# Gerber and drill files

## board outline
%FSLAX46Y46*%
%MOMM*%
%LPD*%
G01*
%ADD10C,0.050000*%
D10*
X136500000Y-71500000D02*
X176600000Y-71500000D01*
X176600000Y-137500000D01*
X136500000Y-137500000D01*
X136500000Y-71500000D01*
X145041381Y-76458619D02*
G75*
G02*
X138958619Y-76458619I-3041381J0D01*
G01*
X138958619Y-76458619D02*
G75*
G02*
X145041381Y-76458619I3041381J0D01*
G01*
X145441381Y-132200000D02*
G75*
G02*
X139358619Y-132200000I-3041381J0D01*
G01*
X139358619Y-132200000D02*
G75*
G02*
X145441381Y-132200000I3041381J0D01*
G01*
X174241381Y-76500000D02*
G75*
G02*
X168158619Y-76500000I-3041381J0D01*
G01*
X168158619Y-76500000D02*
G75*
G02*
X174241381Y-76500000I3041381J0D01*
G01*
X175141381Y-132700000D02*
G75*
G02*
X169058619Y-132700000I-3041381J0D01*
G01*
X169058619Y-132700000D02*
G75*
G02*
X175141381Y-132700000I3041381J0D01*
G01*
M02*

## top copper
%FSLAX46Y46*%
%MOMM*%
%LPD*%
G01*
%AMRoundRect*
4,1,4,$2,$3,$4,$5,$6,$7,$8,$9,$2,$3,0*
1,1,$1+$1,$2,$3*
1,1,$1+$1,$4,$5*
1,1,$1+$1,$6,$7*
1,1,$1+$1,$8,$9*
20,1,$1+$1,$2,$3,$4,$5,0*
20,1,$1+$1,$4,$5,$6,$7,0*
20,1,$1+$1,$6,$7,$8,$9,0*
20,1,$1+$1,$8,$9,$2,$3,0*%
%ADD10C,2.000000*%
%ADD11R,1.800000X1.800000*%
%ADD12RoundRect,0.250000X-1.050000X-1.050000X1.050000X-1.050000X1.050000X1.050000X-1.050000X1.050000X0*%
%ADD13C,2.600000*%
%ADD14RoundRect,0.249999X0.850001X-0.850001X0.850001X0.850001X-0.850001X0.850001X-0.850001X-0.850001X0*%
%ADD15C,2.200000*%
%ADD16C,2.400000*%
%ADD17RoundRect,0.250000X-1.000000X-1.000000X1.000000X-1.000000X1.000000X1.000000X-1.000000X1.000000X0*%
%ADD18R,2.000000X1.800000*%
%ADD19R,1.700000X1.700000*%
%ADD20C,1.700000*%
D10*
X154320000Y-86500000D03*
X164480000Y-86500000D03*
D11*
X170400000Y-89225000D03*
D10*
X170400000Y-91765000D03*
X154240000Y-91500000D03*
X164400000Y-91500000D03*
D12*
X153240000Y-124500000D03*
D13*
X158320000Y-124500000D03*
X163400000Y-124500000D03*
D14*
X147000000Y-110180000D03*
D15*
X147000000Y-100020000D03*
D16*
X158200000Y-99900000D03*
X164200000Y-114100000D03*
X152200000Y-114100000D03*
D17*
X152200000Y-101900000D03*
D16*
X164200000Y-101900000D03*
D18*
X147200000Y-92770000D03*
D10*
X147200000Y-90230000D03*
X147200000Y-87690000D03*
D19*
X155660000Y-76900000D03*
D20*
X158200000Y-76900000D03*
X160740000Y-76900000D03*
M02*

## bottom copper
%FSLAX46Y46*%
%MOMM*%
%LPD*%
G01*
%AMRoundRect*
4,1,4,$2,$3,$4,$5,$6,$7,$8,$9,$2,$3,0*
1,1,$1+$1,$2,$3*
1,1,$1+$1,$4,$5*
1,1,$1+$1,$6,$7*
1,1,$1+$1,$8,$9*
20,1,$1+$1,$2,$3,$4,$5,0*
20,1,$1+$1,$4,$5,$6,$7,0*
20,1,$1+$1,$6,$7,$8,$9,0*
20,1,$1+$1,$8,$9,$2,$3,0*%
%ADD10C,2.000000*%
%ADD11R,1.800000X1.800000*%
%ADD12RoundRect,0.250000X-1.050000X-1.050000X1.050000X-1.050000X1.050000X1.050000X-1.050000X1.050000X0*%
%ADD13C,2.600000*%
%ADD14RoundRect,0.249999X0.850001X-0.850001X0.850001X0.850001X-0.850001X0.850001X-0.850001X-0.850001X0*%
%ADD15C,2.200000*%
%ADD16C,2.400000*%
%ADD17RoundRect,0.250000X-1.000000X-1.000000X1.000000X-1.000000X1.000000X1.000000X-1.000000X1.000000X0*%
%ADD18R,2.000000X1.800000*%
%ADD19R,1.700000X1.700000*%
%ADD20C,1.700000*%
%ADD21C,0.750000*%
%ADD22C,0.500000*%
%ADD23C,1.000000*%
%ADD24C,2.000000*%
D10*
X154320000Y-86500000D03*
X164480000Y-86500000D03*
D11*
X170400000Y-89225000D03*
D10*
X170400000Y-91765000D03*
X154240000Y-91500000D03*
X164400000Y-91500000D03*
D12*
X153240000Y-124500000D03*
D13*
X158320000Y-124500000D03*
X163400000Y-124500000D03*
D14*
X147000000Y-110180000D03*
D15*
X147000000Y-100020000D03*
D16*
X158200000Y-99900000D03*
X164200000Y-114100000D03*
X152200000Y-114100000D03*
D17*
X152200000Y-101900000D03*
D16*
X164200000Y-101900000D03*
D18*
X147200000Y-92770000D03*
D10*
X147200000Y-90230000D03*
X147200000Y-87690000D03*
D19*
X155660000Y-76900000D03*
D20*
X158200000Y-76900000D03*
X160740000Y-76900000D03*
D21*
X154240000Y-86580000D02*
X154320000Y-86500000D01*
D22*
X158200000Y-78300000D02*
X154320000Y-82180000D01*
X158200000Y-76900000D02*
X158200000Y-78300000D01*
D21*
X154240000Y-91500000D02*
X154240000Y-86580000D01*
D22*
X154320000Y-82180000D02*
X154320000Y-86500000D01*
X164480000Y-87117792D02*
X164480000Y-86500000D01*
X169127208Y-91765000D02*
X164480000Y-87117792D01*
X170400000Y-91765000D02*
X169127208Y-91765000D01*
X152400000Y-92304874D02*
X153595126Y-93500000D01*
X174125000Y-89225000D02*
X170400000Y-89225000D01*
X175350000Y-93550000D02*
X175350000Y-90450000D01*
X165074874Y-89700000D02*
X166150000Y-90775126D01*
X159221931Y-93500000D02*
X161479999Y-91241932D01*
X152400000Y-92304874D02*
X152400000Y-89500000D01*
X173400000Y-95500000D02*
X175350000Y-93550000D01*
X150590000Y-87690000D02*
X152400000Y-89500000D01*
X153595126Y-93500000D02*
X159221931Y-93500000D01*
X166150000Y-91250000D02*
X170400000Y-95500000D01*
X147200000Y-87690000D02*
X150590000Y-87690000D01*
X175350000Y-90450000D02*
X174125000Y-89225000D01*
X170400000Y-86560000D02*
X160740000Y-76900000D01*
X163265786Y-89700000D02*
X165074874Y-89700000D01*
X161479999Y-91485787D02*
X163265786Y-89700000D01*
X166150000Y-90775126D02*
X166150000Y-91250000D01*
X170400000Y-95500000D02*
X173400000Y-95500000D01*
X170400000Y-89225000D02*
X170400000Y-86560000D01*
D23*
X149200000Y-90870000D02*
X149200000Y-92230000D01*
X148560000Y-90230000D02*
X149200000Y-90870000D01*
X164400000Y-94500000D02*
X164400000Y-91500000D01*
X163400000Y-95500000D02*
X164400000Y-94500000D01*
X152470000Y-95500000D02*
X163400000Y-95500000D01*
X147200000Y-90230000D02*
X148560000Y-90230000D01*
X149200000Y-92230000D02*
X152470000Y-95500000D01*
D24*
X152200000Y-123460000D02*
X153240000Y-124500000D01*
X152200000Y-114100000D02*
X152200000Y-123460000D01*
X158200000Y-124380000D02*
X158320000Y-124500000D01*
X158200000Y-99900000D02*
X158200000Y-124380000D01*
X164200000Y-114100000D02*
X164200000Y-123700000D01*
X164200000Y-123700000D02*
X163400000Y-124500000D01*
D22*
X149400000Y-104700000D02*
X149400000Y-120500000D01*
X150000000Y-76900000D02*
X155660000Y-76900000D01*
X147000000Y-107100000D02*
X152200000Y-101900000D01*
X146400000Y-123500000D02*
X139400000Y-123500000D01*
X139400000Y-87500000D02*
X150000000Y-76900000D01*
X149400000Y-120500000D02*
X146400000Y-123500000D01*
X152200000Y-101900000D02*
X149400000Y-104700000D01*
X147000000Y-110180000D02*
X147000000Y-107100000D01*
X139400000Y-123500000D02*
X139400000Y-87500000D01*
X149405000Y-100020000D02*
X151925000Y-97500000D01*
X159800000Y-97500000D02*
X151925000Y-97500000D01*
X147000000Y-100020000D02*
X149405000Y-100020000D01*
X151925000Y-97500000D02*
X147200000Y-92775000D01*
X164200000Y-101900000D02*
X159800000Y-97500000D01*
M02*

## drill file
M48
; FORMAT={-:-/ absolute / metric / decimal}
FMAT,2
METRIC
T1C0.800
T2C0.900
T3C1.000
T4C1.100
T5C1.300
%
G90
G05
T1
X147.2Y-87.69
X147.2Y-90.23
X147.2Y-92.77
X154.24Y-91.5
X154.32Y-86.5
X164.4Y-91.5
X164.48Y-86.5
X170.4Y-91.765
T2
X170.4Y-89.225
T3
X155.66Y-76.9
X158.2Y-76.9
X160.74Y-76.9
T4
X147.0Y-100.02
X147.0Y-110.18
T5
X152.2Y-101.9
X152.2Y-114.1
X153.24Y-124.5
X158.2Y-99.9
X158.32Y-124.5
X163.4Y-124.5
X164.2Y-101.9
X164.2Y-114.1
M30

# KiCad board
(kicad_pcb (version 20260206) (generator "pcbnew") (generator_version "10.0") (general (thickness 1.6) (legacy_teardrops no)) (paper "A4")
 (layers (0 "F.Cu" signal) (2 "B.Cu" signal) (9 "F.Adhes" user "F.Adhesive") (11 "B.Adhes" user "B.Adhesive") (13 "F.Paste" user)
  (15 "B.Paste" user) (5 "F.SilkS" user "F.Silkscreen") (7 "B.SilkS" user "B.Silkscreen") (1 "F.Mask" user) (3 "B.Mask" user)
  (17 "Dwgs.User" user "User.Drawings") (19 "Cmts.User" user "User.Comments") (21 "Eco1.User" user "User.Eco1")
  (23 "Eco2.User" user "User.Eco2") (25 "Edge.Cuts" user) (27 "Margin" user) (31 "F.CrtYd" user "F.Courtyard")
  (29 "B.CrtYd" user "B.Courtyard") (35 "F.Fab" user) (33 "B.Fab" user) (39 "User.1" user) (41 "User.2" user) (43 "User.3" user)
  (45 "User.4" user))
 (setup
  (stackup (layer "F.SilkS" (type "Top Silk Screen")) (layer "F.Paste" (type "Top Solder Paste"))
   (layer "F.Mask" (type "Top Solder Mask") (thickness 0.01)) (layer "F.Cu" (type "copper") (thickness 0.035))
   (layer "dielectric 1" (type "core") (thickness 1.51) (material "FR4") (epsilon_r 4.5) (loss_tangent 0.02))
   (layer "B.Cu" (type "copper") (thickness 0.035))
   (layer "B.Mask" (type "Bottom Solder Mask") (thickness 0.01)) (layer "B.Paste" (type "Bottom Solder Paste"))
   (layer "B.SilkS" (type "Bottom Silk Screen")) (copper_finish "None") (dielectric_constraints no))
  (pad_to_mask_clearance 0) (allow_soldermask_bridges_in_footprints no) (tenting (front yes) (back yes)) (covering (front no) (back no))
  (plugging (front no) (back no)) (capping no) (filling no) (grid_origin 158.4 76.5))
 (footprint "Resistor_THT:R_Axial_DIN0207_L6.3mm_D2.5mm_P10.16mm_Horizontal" (layer "F.Cu") (at 154.32 86.5)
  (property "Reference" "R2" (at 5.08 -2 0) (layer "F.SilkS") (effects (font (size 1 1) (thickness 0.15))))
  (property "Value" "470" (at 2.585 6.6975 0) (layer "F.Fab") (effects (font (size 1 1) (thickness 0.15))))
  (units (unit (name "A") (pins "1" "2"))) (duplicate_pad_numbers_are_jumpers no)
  (pad "1" thru_hole circle (at 0 0) (size 2 2) (drill 0.8) (layers "*.Cu" "*.Mask") (remove_unused_layers no) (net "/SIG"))
  (pad "2" thru_hole circle (at 10.16 0) (size 2 2) (drill 0.8) (layers "*.Cu" "*.Mask") (remove_unused_layers no) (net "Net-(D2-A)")))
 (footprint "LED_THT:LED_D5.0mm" (layer "F.Cu") (at 170.4 89.225 -90)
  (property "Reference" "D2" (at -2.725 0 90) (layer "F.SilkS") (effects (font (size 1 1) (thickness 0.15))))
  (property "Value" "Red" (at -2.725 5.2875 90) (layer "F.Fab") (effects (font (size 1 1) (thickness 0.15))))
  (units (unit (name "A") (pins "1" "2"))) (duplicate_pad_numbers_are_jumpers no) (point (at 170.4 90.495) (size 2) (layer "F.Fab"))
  (pad "1" thru_hole rect (at 0 0 270) (size 1.8 1.8) (drill 0.9) (layers "*.Cu" "*.Mask") (remove_unused_layers no) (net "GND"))
  (pad "2" thru_hole circle (at 2.54 0 270) (size 2 2) (drill 0.8) (layers "*.Cu" "*.Mask") (remove_unused_layers no) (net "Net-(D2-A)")))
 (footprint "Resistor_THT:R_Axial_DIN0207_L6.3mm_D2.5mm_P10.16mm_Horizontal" (layer "F.Cu") (at 154.24 91.5)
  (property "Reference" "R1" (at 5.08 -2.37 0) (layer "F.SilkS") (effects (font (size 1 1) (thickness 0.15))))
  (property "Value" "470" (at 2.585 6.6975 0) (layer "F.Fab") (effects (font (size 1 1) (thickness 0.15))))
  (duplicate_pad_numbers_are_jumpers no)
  (pad "1" thru_hole circle (at 0 0) (size 2 2) (drill 0.8) (layers "*.Cu" "*.Mask") (remove_unused_layers no) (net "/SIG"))
  (pad "2" thru_hole circle (at 10.16 0) (size 2 2) (drill 0.8) (layers "*.Cu" "*.Mask") (remove_unused_layers no) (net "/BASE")))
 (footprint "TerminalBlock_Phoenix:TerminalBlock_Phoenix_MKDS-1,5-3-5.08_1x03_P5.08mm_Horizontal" (layer "F.Cu") (at 153.24 124.5)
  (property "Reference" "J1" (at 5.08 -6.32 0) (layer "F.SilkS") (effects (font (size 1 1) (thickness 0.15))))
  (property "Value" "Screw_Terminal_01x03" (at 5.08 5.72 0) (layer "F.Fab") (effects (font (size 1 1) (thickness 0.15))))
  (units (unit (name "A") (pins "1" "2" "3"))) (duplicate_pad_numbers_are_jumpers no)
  (pad "1" thru_hole roundrect (at 0 0) (size 2.6 2.6) (drill 1.3) (layers "*.Cu" "*.Mask") (remove_unused_layers no)
   (roundrect_rratio 0.096154) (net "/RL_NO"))
  (pad "2" thru_hole circle (at 5.08 0) (size 2.6 2.6) (drill 1.3) (layers "*.Cu" "*.Mask") (remove_unused_layers no) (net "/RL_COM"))
  (pad "3" thru_hole circle (at 10.16 0) (size 2.6 2.6) (drill 1.3) (layers "*.Cu" "*.Mask") (remove_unused_layers no) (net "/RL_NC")))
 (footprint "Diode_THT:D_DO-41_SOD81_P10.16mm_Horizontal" (layer "F.Cu") (at 147 110.18 90)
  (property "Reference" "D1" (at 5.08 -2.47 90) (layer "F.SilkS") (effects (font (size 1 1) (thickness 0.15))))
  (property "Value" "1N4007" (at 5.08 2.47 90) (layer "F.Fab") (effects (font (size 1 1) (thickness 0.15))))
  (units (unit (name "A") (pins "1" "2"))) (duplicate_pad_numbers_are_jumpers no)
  (pad "1" thru_hole roundrect (at 0 0 90) (size 2.2 2.2) (drill 1.1) (layers "*.Cu" "*.Mask") (remove_unused_layers no)
   (roundrect_rratio 0.113636) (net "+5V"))
  (pad "2" thru_hole circle (at 10.16 0 90) (size 2.2 2.2) (drill 1.1) (layers "*.Cu" "*.Mask") (remove_unused_layers no) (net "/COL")))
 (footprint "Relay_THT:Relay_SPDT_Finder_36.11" (layer "F.Cu") (at 152.2 101.9)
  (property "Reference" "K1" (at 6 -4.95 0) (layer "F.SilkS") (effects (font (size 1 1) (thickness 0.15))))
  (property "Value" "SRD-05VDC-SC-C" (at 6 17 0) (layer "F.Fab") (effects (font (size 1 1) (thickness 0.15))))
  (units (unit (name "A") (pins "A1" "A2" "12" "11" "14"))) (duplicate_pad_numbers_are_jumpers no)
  (pad "11" thru_hole circle (at 6 -2) (size 2.4 2.4) (drill 1.3) (layers "*.Cu" "*.Mask") (remove_unused_layers no) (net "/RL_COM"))
  (pad "12" thru_hole circle (at 12 12.2) (size 2.4 2.4) (drill 1.3) (layers "*.Cu" "*.Mask") (remove_unused_layers no) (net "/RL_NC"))
  (pad "14" thru_hole circle (at 0 12.2) (size 2.4 2.4) (drill 1.3) (layers "*.Cu" "*.Mask") (remove_unused_layers no) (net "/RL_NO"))
  (pad "A1" thru_hole roundrect (at 0 0) (size 2.5 2.5) (drill 1.3) (layers "*.Cu" "*.Mask") (remove_unused_layers no)
   (roundrect_rratio 0.1) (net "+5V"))
  (pad "A2" thru_hole circle (at 12 0) (size 2.4 2.4) (drill 1.3) (layers "*.Cu" "*.Mask") (remove_unused_layers no) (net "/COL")))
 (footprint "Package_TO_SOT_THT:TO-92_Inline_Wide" (layer "F.Cu") (at 147.2 92.77 90)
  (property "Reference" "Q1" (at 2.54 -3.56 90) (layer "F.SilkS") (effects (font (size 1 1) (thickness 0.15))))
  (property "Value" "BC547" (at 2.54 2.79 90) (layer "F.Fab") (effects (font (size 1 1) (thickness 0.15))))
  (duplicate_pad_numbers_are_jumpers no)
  (pad "1" thru_hole rect (at 0 0 90) (size 1.8 2) (drill 0.8) (layers "*.Cu" "*.Mask") (remove_unused_layers no) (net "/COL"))
  (pad "2" thru_hole circle (at 2.54 0 90) (size 2 2) (drill 0.8) (layers "*.Cu" "*.Mask") (remove_unused_layers no) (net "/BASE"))
  (pad "3" thru_hole circle (at 5.08 0 90) (size 2 2) (drill 0.8) (layers "*.Cu" "*.Mask") (remove_unused_layers no) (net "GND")))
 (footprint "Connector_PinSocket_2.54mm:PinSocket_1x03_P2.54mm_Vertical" (layer "F.Cu") (at 155.66 76.9 90)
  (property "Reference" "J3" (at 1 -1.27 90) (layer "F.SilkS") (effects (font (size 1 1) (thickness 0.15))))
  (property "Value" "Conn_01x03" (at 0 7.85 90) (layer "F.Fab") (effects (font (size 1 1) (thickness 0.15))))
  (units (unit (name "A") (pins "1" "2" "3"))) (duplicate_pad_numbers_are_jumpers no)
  (pad "1" thru_hole rect (at 0 0 90) (size 1.7 1.7) (drill 1) (layers "*.Cu" "*.Mask") (remove_unused_layers no) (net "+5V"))
  (pad "2" thru_hole circle (at 0 2.54 90) (size 1.7 1.7) (drill 1) (layers "*.Cu" "*.Mask") (remove_unused_layers no) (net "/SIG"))
  (pad "3" thru_hole circle (at 0 5.08 90) (size 1.7 1.7) (drill 1) (layers "*.Cu" "*.Mask") (remove_unused_layers no) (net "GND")))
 (gr_rect (start 136.5 71.5) (end 176.6 137.5) (stroke (width 0.05) (type default)) (fill no) (layer "Edge.Cuts"))
 (gr_circle (center 142 76.458619) (end 141.5 73.458619) (stroke (width 0.05) (type default)) (fill no) (layer "Edge.Cuts"))
 (gr_circle (center 142.4 132.2) (end 141.9 129.2) (stroke (width 0.05) (type default)) (fill no) (layer "Edge.Cuts"))
 (gr_circle (center 171.2 76.5) (end 170.7 73.5) (stroke (width 0.05) (type default)) (fill no) (layer "Edge.Cuts"))
 (gr_circle (center 172.1 132.7) (end 171.6 129.7) (stroke (width 0.05) (type default)) (fill no) (layer "Edge.Cuts"))
 (segment (start 154.24 86.58) (end 154.32 86.5) (width 0.75) (layer "B.Cu") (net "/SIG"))
 (segment (start 158.2 78.3) (end 154.32 82.18) (width 0.5) (layer "B.Cu") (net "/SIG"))
 (segment (start 158.2 76.9) (end 158.2 78.3) (width 0.5) (layer "B.Cu") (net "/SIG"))
 (segment (start 154.24 91.5) (end 154.24 86.58) (width 0.75) (layer "B.Cu") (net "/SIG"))
 (segment (start 154.32 82.18) (end 154.32 86.5) (width 0.5) (layer "B.Cu") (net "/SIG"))
 (segment (start 164.48 87.117792) (end 164.48 86.5) (width 0.5) (layer "B.Cu") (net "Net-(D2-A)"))
 (segment (start 169.127208 91.765) (end 164.48 87.117792) (width 0.5) (layer "B.Cu") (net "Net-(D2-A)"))
 (segment (start 170.4 91.765) (end 169.127208 91.765) (width 0.5) (layer "B.Cu") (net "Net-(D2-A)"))
 (segment (start 152.4 92.304874) (end 153.595126 93.5) (width 0.5) (layer "B.Cu") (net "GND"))
 (segment (start 174.125 89.225) (end 170.4 89.225) (width 0.5) (layer "B.Cu") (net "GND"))
 (segment (start 175.35 93.55) (end 175.35 90.45) (width 0.5) (layer "B.Cu") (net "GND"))
 (segment (start 165.074874 89.7) (end 166.15 90.775126) (width 0.5) (layer "B.Cu") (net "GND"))
 (segment (start 159.221931 93.5) (end 161.479999 91.241932) (width 0.5) (layer "B.Cu") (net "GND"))
 (segment (start 152.4 92.304874) (end 152.4 89.5) (width 0.5) (layer "B.Cu") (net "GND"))
 (segment (start 173.4 95.5) (end 175.35 93.55) (width 0.5) (layer "B.Cu") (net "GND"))
 (segment (start 150.59 87.69) (end 152.4 89.5) (width 0.5) (layer "B.Cu") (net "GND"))
 (segment (start 153.595126 93.5) (end 159.221931 93.5) (width 0.5) (layer "B.Cu") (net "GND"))
 (segment (start 166.15 91.25) (end 170.4 95.5) (width 0.5) (layer "B.Cu") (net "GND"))
 (segment (start 147.2 87.69) (end 150.59 87.69) (width 0.5) (layer "B.Cu") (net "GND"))
 (segment (start 175.35 90.45) (end 174.125 89.225) (width 0.5) (layer "B.Cu") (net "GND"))
 (segment (start 170.4 86.56) (end 160.74 76.9) (width 0.5) (layer "B.Cu") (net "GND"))
 (segment (start 163.265786 89.7) (end 165.074874 89.7) (width 0.5) (layer "B.Cu") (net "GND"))
 (segment (start 161.479999 91.485787) (end 163.265786 89.7) (width 0.5) (layer "B.Cu") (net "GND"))
 (segment (start 166.15 90.775126) (end 166.15 91.25) (width 0.5) (layer "B.Cu") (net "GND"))
 (segment (start 170.4 95.5) (end 173.4 95.5) (width 0.5) (layer "B.Cu") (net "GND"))
 (segment (start 170.4 89.225) (end 170.4 86.56) (width 0.5) (layer "B.Cu") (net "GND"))
 (segment (start 149.2 90.87) (end 149.2 92.23) (width 1) (layer "B.Cu") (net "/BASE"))
 (segment (start 148.56 90.23) (end 149.2 90.87) (width 1) (layer "B.Cu") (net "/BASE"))
 (segment (start 164.4 94.5) (end 164.4 91.5) (width 1) (layer "B.Cu") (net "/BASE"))
 (segment (start 163.4 95.5) (end 164.4 94.5) (width 1) (layer "B.Cu") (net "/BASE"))
 (segment (start 152.47 95.5) (end 163.4 95.5) (width 1) (layer "B.Cu") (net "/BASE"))
 (segment (start 147.2 90.23) (end 148.56 90.23) (width 1) (layer "B.Cu") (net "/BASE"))
 (segment (start 149.2 92.23) (end 152.47 95.5) (width 1) (layer "B.Cu") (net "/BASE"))
 (segment (start 152.2 123.46) (end 153.24 124.5) (width 2) (layer "B.Cu") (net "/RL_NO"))
 (segment (start 152.2 114.1) (end 152.2 123.46) (width 2) (layer "B.Cu") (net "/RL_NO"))
 (segment (start 158.2 124.38) (end 158.32 124.5) (width 2) (layer "B.Cu") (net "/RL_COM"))
 (segment (start 158.2 99.9) (end 158.2 124.38) (width 2) (layer "B.Cu") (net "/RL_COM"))
 (segment (start 164.2 114.1) (end 164.2 123.7) (width 2) (layer "B.Cu") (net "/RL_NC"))
 (segment (start 164.2 123.7) (end 163.4 124.5) (width 2) (layer "B.Cu") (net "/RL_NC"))
 (segment (start 149.4 104.7) (end 149.4 120.5) (width 0.5) (layer "B.Cu") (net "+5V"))
 (segment (start 150 76.9) (end 155.66 76.9) (width 0.5) (layer "B.Cu") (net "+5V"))
 (segment (start 147 107.1) (end 152.2 101.9) (width 0.5) (layer "B.Cu") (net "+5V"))
 (segment (start 146.4 123.5) (end 139.4 123.5) (width 0.5) (layer "B.Cu") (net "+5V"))
 (segment (start 139.4 87.5) (end 150 76.9) (width 0.5) (layer "B.Cu") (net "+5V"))
 (segment (start 149.4 120.5) (end 146.4 123.5) (width 0.5) (layer "B.Cu") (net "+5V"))
 (segment (start 152.2 101.9) (end 149.4 104.7) (width 0.5) (layer "B.Cu") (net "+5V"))
 (segment (start 147 110.18) (end 147 107.1) (width 0.5) (layer "B.Cu") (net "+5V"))
 (segment (start 139.4 123.5) (end 139.4 87.5) (width 0.5) (layer "B.Cu") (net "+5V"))
 (segment (start 149.405 100.02) (end 151.925 97.5) (width 0.5) (layer "B.Cu") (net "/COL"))
 (segment (start 159.8 97.5) (end 151.925 97.5) (width 0.5) (layer "B.Cu") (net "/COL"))
 (segment (start 147 100.02) (end 149.405 100.02) (width 0.5) (layer "B.Cu") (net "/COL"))
 (segment (start 151.925 97.5) (end 147.2 92.775) (width 0.5) (layer "B.Cu") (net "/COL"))
 (segment (start 164.2 101.9) (end 159.8 97.5) (width 0.5) (layer "B.Cu") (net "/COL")))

